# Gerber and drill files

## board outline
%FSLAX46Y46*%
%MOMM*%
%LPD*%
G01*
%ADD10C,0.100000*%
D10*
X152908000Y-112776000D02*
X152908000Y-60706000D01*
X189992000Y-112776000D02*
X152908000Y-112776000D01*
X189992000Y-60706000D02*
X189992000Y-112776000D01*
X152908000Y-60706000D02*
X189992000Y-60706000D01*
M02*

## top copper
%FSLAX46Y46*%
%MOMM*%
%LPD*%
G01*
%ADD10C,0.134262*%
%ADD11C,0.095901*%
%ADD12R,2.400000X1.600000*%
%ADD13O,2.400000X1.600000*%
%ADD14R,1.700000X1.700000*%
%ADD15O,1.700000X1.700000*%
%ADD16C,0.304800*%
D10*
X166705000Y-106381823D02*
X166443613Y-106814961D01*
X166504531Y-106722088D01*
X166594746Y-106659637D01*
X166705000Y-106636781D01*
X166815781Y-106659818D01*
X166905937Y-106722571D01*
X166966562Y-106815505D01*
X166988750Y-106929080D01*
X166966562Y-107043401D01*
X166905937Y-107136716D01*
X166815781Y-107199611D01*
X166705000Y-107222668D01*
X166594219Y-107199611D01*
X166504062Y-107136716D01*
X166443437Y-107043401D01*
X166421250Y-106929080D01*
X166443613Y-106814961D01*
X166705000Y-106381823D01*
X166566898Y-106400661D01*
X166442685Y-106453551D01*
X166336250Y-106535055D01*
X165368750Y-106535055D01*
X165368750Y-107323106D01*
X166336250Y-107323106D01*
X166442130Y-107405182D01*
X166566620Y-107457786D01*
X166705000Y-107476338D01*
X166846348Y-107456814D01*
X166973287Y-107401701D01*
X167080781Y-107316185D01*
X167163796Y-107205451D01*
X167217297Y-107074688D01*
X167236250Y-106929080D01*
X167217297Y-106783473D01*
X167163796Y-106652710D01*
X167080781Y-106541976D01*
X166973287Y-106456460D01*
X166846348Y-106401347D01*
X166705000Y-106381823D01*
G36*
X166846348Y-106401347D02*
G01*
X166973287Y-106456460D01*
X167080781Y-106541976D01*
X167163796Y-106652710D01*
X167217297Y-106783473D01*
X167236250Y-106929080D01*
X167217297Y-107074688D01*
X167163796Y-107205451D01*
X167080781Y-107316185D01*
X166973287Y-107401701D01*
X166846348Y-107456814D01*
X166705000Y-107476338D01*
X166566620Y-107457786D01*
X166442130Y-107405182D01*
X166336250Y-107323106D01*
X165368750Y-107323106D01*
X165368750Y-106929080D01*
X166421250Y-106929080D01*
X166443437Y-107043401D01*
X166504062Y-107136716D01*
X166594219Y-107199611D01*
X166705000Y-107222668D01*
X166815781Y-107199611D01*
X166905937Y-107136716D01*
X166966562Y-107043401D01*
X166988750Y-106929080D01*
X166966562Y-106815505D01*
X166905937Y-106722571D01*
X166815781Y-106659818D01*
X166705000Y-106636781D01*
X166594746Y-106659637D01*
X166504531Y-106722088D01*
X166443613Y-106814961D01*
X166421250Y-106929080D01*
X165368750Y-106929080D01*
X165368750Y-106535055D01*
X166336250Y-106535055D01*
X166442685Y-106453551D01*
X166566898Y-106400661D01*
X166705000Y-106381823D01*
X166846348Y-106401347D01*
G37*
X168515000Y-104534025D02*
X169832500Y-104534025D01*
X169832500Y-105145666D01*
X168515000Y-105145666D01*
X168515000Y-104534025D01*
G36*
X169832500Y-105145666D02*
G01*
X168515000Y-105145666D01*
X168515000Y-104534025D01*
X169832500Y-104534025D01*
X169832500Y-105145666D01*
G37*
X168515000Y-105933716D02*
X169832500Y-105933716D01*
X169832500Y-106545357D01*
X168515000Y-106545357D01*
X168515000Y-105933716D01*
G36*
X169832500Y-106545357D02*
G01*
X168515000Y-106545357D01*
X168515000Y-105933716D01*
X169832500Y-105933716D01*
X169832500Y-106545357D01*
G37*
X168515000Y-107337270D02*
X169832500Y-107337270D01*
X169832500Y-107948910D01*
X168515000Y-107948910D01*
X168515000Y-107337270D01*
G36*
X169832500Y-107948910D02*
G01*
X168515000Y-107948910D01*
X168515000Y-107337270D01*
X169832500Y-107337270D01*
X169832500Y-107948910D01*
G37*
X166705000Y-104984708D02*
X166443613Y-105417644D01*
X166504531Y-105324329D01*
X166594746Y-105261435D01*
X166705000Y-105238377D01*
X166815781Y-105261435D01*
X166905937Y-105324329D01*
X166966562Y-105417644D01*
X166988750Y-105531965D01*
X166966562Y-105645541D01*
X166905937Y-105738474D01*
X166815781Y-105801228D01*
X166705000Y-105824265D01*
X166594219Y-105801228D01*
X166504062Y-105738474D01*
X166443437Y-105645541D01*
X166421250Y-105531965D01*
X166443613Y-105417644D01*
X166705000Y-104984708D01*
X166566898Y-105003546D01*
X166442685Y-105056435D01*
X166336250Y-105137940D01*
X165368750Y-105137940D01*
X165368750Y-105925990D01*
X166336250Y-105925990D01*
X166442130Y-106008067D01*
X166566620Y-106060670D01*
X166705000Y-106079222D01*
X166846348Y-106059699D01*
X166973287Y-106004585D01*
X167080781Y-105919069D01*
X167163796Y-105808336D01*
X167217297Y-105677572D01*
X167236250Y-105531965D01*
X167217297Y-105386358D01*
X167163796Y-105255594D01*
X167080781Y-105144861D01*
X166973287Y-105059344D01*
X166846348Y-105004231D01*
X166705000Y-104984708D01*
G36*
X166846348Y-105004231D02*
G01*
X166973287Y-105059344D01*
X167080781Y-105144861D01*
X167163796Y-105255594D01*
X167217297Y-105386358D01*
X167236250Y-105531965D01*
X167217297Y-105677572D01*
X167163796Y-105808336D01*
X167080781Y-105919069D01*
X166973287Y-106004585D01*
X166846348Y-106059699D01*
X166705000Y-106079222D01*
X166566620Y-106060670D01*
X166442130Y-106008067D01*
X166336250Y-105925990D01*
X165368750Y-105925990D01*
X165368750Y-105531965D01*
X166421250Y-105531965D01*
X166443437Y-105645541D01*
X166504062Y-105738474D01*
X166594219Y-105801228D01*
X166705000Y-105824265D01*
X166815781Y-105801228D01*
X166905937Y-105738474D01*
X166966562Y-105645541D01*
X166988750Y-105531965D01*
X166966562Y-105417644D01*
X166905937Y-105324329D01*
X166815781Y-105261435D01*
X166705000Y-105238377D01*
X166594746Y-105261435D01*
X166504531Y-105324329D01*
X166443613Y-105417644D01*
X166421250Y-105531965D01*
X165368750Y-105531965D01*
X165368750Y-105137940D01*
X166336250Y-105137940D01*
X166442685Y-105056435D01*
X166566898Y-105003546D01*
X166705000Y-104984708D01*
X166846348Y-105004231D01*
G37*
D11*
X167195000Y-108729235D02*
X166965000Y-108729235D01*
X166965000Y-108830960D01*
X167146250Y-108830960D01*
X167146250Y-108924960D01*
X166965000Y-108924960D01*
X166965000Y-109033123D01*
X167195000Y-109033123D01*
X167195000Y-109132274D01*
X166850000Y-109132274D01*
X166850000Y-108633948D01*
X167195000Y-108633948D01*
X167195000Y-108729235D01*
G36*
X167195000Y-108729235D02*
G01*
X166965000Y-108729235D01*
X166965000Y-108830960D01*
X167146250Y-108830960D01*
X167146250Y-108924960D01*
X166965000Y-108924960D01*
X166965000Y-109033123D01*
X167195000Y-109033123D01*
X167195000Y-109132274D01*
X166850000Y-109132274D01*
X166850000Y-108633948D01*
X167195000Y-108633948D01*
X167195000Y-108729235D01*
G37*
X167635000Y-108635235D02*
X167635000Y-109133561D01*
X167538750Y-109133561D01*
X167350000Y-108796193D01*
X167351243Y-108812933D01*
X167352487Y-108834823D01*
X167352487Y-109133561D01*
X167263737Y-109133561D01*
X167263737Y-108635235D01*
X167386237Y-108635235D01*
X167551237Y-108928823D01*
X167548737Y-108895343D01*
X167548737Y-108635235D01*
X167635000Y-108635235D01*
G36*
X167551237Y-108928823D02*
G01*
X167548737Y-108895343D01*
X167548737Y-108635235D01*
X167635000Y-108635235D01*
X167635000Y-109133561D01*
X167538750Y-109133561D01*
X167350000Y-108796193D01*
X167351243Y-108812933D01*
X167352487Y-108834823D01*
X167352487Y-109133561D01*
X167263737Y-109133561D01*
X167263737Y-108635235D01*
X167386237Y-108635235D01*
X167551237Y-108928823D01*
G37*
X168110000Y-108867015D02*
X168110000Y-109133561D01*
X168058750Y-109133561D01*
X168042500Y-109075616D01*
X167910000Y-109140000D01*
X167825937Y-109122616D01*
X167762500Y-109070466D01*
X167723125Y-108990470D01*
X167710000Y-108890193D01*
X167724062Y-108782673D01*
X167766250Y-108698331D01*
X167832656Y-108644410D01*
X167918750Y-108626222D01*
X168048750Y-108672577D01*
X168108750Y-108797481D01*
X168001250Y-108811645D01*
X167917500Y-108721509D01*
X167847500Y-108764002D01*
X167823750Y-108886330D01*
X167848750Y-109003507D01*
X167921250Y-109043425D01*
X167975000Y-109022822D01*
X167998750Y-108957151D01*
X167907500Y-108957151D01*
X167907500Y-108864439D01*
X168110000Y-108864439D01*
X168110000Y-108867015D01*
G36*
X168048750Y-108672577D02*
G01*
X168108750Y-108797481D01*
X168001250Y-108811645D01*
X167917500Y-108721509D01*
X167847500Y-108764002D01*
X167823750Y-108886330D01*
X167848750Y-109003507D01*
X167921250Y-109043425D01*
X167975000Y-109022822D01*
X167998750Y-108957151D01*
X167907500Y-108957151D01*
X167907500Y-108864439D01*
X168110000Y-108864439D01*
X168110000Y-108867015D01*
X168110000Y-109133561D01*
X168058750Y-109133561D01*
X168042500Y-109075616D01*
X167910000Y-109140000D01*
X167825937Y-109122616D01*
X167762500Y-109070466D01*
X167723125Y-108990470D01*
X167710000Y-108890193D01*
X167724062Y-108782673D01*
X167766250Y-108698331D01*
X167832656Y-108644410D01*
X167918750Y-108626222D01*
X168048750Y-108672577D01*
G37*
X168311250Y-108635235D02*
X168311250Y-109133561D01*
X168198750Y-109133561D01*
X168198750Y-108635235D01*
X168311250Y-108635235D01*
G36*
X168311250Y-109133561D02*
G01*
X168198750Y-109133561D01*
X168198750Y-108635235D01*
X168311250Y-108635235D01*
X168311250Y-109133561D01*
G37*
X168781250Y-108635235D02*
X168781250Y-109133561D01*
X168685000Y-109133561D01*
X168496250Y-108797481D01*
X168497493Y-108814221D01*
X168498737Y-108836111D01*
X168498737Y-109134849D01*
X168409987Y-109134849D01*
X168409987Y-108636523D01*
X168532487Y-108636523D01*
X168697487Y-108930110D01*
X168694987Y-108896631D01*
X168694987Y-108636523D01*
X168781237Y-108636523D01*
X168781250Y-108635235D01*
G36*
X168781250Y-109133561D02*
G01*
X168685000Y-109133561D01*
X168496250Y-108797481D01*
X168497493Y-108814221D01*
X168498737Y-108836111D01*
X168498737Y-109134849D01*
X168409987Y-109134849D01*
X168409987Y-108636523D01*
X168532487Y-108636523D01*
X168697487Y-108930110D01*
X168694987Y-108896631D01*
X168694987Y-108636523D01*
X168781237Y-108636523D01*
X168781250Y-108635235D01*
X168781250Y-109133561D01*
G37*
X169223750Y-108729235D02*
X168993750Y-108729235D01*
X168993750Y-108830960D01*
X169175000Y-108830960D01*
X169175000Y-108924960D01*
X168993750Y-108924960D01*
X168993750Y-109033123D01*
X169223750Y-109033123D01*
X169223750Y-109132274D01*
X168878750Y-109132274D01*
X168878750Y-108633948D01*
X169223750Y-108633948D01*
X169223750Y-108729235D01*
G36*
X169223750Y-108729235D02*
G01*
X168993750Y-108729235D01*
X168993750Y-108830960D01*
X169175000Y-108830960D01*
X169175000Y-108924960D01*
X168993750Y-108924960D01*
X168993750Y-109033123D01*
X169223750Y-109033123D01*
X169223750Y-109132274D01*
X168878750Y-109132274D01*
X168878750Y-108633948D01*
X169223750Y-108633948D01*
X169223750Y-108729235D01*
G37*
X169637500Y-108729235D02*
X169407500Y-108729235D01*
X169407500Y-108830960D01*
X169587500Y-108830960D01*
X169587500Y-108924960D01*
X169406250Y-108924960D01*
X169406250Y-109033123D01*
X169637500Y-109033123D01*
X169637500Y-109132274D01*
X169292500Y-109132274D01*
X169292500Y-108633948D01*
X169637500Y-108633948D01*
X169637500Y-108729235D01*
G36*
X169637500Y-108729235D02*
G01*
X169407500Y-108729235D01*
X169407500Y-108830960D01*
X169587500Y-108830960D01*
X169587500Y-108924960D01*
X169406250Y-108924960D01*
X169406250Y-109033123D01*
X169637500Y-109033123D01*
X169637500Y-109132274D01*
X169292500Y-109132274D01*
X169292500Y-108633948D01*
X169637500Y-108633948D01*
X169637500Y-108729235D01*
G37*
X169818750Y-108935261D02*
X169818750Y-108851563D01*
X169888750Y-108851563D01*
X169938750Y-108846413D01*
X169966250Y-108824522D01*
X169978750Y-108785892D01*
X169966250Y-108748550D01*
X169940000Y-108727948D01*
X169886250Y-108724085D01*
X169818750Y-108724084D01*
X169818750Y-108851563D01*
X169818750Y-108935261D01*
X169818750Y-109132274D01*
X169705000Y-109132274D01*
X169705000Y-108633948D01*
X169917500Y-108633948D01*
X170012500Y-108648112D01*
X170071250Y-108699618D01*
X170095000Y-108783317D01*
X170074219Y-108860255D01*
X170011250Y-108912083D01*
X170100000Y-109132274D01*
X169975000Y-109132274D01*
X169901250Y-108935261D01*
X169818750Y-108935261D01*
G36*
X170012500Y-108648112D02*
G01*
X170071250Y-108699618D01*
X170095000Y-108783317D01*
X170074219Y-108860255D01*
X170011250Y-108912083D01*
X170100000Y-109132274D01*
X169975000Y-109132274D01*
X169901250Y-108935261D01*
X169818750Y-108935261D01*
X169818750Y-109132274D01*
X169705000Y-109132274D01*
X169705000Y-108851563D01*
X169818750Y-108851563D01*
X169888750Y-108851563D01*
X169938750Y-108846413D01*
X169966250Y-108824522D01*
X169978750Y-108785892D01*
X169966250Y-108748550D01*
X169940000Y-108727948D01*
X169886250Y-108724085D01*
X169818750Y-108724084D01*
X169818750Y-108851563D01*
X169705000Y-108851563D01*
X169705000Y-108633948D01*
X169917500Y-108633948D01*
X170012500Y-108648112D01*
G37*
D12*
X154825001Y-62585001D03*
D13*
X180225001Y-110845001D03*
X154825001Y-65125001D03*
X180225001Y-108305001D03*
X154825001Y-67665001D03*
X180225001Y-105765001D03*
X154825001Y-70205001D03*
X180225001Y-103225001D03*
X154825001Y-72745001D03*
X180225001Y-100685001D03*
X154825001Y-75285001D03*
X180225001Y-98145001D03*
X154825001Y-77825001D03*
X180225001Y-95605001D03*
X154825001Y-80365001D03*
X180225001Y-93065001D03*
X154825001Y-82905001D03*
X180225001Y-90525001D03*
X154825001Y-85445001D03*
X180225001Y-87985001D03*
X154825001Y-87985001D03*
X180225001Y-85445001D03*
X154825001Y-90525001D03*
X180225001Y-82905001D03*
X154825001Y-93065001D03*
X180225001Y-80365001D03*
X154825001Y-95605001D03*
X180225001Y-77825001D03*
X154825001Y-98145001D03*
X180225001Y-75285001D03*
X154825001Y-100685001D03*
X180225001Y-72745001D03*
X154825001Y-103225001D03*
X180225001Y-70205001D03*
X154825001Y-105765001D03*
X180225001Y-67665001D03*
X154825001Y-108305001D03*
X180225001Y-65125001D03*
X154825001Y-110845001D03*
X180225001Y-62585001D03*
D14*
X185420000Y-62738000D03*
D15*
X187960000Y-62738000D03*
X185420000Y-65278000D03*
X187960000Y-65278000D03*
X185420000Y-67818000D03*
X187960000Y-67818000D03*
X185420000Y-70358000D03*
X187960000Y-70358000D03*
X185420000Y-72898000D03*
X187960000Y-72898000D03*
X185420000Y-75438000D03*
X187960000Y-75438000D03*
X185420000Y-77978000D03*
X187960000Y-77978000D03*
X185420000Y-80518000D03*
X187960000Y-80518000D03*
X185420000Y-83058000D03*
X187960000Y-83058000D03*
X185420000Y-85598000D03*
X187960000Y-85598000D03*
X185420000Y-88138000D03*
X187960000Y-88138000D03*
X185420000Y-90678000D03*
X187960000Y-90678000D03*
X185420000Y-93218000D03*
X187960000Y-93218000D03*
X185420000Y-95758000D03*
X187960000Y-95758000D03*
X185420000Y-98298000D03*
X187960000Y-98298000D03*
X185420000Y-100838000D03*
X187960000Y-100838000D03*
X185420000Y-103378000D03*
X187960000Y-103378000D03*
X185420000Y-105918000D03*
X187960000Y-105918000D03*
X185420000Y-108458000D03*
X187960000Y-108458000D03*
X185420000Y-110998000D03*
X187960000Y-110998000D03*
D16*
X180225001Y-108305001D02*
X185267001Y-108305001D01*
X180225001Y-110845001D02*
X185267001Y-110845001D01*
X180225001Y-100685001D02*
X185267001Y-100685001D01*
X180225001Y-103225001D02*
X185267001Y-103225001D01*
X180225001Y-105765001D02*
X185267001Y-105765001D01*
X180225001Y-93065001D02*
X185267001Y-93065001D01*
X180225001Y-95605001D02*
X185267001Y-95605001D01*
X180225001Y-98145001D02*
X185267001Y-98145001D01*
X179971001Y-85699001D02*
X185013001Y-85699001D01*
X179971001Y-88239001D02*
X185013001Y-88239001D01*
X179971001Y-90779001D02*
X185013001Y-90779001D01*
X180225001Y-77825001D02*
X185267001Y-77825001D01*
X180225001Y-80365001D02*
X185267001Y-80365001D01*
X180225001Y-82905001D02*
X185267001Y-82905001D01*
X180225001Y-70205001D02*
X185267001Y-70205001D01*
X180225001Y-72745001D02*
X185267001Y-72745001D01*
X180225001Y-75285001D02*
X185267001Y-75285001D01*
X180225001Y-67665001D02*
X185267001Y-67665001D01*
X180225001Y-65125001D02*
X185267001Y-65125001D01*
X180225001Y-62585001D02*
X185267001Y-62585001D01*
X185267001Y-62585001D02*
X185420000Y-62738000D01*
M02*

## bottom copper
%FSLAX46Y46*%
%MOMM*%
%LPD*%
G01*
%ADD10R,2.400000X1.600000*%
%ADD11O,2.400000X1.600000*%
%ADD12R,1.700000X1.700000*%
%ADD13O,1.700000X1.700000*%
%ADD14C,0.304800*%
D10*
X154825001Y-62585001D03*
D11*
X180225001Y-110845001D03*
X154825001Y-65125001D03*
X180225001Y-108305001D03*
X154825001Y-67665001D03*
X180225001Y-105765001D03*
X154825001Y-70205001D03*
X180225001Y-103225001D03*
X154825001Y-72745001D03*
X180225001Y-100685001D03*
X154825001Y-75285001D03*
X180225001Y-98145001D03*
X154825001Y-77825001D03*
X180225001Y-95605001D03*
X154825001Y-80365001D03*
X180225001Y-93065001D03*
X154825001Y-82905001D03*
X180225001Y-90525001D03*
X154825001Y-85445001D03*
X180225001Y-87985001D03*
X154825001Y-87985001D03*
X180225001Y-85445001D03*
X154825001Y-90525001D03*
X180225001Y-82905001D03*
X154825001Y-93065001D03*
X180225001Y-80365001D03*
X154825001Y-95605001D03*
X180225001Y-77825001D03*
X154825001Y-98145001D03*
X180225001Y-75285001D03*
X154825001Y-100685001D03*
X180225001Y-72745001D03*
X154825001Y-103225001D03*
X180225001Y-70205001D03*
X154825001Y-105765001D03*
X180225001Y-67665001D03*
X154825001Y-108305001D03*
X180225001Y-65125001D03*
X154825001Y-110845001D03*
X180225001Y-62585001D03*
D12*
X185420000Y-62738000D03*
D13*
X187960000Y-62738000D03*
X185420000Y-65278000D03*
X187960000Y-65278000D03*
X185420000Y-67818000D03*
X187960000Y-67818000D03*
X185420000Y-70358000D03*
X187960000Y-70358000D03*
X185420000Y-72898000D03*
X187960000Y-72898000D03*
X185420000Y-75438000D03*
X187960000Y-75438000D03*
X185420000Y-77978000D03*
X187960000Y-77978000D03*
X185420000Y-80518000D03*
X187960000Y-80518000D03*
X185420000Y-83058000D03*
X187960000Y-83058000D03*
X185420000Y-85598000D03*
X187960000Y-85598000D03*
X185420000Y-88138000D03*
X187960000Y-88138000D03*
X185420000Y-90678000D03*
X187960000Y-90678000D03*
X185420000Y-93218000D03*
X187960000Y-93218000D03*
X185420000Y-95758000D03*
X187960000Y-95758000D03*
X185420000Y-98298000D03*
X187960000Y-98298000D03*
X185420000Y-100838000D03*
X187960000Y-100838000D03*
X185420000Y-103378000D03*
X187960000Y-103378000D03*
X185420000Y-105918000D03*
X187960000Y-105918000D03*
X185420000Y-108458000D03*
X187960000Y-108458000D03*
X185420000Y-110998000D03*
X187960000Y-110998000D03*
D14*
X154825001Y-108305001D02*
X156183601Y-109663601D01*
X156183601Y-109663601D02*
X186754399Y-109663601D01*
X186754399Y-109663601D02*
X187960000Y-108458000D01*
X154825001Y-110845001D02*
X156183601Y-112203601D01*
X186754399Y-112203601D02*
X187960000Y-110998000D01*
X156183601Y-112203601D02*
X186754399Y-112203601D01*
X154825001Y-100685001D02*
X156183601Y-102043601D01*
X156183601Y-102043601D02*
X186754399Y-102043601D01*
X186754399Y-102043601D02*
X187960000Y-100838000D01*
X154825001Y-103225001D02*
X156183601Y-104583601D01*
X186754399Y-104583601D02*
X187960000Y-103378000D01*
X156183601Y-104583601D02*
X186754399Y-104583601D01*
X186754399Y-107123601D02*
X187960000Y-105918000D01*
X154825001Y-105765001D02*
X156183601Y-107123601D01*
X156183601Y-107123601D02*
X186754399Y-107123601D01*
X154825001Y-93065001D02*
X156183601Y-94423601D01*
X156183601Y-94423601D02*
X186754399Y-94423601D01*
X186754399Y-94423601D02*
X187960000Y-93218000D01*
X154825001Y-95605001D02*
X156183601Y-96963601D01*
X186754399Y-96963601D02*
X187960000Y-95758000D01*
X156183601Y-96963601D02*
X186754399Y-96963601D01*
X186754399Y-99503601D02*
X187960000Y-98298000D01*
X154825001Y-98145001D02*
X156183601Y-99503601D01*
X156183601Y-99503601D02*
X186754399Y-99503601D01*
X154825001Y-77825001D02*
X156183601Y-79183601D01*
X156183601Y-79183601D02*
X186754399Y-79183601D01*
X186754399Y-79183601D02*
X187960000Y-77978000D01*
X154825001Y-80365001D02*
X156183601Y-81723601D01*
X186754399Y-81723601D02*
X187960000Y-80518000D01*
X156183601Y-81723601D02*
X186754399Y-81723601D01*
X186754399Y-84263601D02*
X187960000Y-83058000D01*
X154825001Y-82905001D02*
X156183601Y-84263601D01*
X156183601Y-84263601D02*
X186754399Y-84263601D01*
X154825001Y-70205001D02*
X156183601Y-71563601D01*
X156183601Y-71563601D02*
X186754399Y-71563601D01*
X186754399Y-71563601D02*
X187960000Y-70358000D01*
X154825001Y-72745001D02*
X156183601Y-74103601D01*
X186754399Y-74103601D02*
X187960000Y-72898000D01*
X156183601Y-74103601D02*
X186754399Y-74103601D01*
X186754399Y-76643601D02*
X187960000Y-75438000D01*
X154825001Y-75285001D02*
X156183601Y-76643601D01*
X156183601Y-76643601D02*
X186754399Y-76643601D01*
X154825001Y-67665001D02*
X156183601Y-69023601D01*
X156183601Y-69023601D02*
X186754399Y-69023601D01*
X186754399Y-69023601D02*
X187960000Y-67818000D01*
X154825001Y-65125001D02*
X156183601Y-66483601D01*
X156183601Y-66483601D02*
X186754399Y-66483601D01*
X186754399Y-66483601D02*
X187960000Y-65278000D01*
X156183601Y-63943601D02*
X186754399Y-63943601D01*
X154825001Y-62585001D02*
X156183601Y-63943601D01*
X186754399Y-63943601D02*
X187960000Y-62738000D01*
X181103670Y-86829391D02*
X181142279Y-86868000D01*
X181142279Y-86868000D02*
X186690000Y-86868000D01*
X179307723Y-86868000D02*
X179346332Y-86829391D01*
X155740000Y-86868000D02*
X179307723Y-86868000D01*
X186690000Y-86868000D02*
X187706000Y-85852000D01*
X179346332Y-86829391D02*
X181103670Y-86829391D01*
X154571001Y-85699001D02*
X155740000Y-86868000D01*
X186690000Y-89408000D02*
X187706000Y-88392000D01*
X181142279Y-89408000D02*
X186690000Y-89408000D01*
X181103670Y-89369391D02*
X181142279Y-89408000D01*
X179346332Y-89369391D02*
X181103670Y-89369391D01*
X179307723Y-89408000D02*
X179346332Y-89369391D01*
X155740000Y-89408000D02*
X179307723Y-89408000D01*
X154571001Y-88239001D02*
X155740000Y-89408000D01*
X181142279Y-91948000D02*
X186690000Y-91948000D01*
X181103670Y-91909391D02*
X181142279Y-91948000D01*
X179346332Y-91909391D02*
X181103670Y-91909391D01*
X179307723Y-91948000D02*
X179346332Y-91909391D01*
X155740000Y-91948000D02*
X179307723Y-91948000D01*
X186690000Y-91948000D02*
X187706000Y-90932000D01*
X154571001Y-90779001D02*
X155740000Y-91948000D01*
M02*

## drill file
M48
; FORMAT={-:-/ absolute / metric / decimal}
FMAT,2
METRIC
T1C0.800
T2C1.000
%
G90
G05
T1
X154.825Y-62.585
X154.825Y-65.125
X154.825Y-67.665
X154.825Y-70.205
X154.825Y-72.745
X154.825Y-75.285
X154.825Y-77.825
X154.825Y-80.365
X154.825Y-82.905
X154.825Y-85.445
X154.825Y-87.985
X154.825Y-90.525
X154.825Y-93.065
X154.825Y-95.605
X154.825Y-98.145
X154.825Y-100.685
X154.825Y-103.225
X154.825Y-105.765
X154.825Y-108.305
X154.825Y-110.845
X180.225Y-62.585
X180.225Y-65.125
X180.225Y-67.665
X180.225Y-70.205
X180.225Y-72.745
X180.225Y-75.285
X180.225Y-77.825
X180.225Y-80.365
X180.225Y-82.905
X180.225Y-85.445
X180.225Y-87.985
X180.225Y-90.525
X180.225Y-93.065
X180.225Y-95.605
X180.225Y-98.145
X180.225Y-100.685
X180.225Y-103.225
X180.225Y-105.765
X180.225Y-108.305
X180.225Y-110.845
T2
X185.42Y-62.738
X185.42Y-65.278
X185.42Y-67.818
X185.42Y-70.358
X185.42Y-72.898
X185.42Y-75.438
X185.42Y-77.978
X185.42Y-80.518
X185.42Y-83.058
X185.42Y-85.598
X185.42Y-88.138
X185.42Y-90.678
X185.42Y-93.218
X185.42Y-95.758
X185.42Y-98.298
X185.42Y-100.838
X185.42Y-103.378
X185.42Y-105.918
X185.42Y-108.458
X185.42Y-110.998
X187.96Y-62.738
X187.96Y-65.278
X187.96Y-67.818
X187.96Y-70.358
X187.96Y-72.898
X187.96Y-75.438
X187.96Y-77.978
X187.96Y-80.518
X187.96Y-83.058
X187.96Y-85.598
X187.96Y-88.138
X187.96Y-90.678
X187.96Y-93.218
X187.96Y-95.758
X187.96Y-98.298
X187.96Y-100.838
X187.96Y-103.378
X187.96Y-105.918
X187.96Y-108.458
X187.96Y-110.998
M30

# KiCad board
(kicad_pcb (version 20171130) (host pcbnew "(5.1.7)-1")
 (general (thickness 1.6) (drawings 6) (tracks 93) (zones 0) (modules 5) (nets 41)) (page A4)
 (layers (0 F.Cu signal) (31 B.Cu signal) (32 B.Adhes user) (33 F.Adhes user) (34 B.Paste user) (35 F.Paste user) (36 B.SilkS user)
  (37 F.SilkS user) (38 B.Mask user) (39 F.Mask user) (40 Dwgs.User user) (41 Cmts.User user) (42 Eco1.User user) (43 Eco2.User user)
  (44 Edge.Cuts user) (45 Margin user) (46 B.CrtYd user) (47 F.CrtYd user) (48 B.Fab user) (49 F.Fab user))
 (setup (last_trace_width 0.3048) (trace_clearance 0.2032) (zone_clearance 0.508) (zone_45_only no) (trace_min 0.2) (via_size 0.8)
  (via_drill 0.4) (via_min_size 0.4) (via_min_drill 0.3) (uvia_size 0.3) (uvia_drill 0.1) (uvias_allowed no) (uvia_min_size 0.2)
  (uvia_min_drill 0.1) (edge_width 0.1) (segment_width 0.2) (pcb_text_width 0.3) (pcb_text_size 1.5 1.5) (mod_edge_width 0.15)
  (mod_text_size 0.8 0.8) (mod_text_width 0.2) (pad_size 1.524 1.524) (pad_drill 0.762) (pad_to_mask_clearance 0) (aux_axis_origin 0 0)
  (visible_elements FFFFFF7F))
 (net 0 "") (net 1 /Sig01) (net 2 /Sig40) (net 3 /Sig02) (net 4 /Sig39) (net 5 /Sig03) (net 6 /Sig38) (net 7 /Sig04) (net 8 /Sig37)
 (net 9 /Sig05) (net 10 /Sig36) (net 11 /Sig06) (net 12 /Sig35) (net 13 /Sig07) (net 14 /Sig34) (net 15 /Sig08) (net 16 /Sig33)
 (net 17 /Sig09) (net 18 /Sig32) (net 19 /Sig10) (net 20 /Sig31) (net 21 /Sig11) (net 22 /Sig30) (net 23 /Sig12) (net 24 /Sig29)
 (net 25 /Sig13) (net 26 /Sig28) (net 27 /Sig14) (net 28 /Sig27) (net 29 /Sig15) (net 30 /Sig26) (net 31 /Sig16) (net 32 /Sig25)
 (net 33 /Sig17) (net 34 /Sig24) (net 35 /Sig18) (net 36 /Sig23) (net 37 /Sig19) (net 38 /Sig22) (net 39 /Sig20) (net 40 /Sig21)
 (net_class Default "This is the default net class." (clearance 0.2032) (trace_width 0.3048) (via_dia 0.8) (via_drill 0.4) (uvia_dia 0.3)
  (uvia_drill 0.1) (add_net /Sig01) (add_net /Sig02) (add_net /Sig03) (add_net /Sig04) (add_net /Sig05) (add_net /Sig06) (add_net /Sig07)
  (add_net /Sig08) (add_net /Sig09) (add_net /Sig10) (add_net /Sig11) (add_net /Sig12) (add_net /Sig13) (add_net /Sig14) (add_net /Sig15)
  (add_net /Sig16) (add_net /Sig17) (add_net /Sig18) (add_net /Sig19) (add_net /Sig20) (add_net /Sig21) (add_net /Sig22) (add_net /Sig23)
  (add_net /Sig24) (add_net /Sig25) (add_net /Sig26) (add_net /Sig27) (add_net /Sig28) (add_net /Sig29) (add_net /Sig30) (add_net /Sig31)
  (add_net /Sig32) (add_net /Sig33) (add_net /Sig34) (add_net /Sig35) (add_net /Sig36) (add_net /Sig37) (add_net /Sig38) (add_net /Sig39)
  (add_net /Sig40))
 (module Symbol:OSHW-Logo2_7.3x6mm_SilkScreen (layer B.Cu) (at 167.386 106.934 180)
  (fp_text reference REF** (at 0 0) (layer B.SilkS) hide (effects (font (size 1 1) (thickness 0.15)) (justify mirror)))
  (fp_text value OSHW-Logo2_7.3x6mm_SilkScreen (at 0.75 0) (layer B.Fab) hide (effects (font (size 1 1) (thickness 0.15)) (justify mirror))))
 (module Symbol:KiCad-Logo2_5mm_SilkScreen (layer B.Cu) (at 167.386 86.614 180)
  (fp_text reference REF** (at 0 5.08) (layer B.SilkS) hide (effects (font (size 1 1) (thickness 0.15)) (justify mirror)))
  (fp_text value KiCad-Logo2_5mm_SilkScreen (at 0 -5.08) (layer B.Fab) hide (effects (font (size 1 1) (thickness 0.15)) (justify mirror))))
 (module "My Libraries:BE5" (layer F.Cu) (at 165.1 104.14)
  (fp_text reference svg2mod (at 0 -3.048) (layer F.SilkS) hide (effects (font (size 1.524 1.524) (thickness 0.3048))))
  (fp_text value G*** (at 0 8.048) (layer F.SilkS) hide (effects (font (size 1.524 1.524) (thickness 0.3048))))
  (fp_poly
   (pts (xy 1.605 2.241823) (xy 1.343613 2.674961) (xy 1.404531 2.582088) (xy 1.494746 2.519637) (xy 1.605 2.496781) (xy 1.715781 2.519818)
    (xy 1.805937 2.582571) (xy 1.866562 2.675505) (xy 1.88875 2.78908) (xy 1.866562 2.903401) (xy 1.805937 2.996716) (xy 1.715781 3.059611)
    (xy 1.605 3.082668) (xy 1.494219 3.059611) (xy 1.404062 2.996716) (xy 1.343437 2.903401) (xy 1.32125 2.78908) (xy 1.343613 2.674961)
    (xy 1.605 2.241823) (xy 1.466898 2.260661) (xy 1.342685 2.313551) (xy 1.23625 2.395055) (xy 0.26875 2.395055) (xy 0.26875 3.183106)
    (xy 1.23625 3.183106) (xy 1.34213 3.265182) (xy 1.46662 3.317786) (xy 1.605 3.336338) (xy 1.746348 3.316814) (xy 1.873287 3.261701)
    (xy 1.980781 3.176185) (xy 2.063796 3.065451) (xy 2.117297 2.934688) (xy 2.13625 2.78908) (xy 2.117297 2.643473) (xy 2.063796 2.51271)
    (xy 1.980781 2.401976) (xy 1.873287 2.31646) (xy 1.746348 2.261347) (xy 1.605 2.241823))
   (layer F.Cu) (width 0.134262))
  (fp_poly
   (pts (xy 3.415 0.394025) (xy 4.7325 0.394025) (xy 4.7325 1.005666) (xy 3.415 1.005666) (xy 3.415 0.394025)) (layer F.Cu) (width 0.134262))
  (fp_poly
   (pts (xy 3.415 1.793716) (xy 4.7325 1.793716) (xy 4.7325 2.405357) (xy 3.415 2.405357) (xy 3.415 1.793716)) (layer F.Cu) (width 0.134262))
  (fp_poly
   (pts (xy 3.415 3.19727) (xy 4.7325 3.19727) (xy 4.7325 3.80891) (xy 3.415 3.80891) (xy 3.415 3.19727)) (layer F.Cu) (width 0.134262))
  (fp_poly
   (pts (xy 1.605 0.844708) (xy 1.343613 1.277644) (xy 1.404531 1.184329) (xy 1.494746 1.121435) (xy 1.605 1.098377) (xy 1.715781 1.121435)
    (xy 1.805937 1.184329) (xy 1.866562 1.277644) (xy 1.88875 1.391965) (xy 1.866562 1.505541) (xy 1.805937 1.598474) (xy 1.715781 1.661228)
    (xy 1.605 1.684265) (xy 1.494219 1.661228) (xy 1.404062 1.598474) (xy 1.343437 1.505541) (xy 1.32125 1.391965) (xy 1.343613 1.277644)
    (xy 1.605 0.844708) (xy 1.466898 0.863546) (xy 1.342685 0.916435) (xy 1.23625 0.99794) (xy 0.26875 0.99794) (xy 0.26875 1.78599)
    (xy 1.23625 1.78599) (xy 1.34213 1.868067) (xy 1.46662 1.92067) (xy 1.605 1.939222) (xy 1.746348 1.919699) (xy 1.873287 1.864585)
    (xy 1.980781 1.779069) (xy 2.063796 1.668336) (xy 2.117297 1.537572) (xy 2.13625 1.391965) (xy 2.117297 1.246358) (xy 2.063796 1.115594)
    (xy 1.980781 1.004861) (xy 1.873287 0.919344) (xy 1.746348 0.864231) (xy 1.605 0.844708))
   (layer F.Cu) (width 0.134262))
  (fp_poly
   (pts (xy 2.095 4.589235) (xy 1.865 4.589235) (xy 1.865 4.69096) (xy 2.04625 4.69096) (xy 2.04625 4.78496) (xy 1.865 4.78496)
    (xy 1.865 4.893123) (xy 2.095 4.893123) (xy 2.095 4.992274) (xy 1.75 4.992274) (xy 1.75 4.493948) (xy 2.095 4.493948)
    (xy 2.095 4.589235))
   (layer F.Cu) (width 0.095901))
  (fp_poly
   (pts (xy 2.535 4.495235) (xy 2.535 4.993561) (xy 2.43875 4.993561) (xy 2.25 4.656193) (xy 2.251243 4.672933) (xy 2.252487 4.694823)
    (xy 2.252487 4.993561) (xy 2.163737 4.993561) (xy 2.163737 4.495235) (xy 2.286237 4.495235) (xy 2.451237 4.788823)
    (xy 2.448737 4.755343) (xy 2.448737 4.495235) (xy 2.535 4.495235))
   (layer F.Cu) (width 0.095901))
  (fp_poly
   (pts (xy 3.01 4.727015) (xy 3.01 4.993561) (xy 2.95875 4.993561) (xy 2.9425 4.935616) (xy 2.81 5) (xy 2.725937 4.982616)
    (xy 2.6625 4.930466) (xy 2.623125 4.85047) (xy 2.61 4.750193) (xy 2.624062 4.642673) (xy 2.66625 4.558331) (xy 2.732656 4.50441)
    (xy 2.81875 4.486222) (xy 2.94875 4.532577) (xy 3.00875 4.657481) (xy 2.90125 4.671645) (xy 2.8175 4.581509) (xy 2.7475 4.624002)
    (xy 2.72375 4.74633) (xy 2.74875 4.863507) (xy 2.82125 4.903425) (xy 2.875 4.882822) (xy 2.89875 4.817151) (xy 2.8075 4.817151)
    (xy 2.8075 4.724439) (xy 3.01 4.724439) (xy 3.01 4.727015))
   (layer F.Cu) (width 0.095901))
  (fp_poly
   (pts (xy 3.21125 4.495235) (xy 3.21125 4.993561) (xy 3.09875 4.993561) (xy 3.09875 4.495235) (xy 3.21125 4.495235)) (layer F.Cu)
   (width 0.095901))
  (fp_poly
   (pts (xy 3.68125 4.495235) (xy 3.68125 4.993561) (xy 3.585 4.993561) (xy 3.39625 4.657481) (xy 3.397493 4.674221) (xy 3.398737 4.696111)
    (xy 3.398737 4.994849) (xy 3.309987 4.994849) (xy 3.309987 4.496523) (xy 3.432487 4.496523) (xy 3.597487 4.79011) (xy 3.594987 4.756631)
    (xy 3.594987 4.496523) (xy 3.681237 4.496523) (xy 3.68125 4.495235))
   (layer F.Cu) (width 0.095901))
  (fp_poly
   (pts (xy 4.12375 4.589235) (xy 3.89375 4.589235) (xy 3.89375 4.69096) (xy 4.075 4.69096) (xy 4.075 4.78496) (xy 3.89375 4.78496)
    (xy 3.89375 4.893123) (xy 4.12375 4.893123) (xy 4.12375 4.992274) (xy 3.77875 4.992274) (xy 3.77875 4.493948) (xy 4.12375 4.493948)
    (xy 4.12375 4.589235))
   (layer F.Cu) (width 0.095901))
  (fp_poly
   (pts (xy 4.5375 4.589235) (xy 4.3075 4.589235) (xy 4.3075 4.69096) (xy 4.4875 4.69096) (xy 4.4875 4.78496) (xy 4.30625 4.78496)
    (xy 4.30625 4.893123) (xy 4.5375 4.893123) (xy 4.5375 4.992274) (xy 4.1925 4.992274) (xy 4.1925 4.493948) (xy 4.5375 4.493948)
    (xy 4.5375 4.589235))
   (layer F.Cu) (width 0.095901))
  (fp_poly
   (pts (xy 4.71875 4.795261) (xy 4.71875 4.711563) (xy 4.78875 4.711563) (xy 4.83875 4.706413) (xy 4.86625 4.684522) (xy 4.87875 4.645892)
    (xy 4.86625 4.60855) (xy 4.84 4.587948) (xy 4.78625 4.584085) (xy 4.71875 4.584084) (xy 4.71875 4.711563) (xy 4.71875 4.795261)
    (xy 4.71875 4.992274) (xy 4.605 4.992274) (xy 4.605 4.493948) (xy 4.8175 4.493948) (xy 4.9125 4.508112) (xy 4.97125 4.559618)
    (xy 4.995 4.643317) (xy 4.974219 4.720255) (xy 4.91125 4.772083) (xy 5 4.992274) (xy 4.875 4.992274) (xy 4.80125 4.795261)
    (xy 4.71875 4.795261))
   (layer F.Cu) (width 0.095901)))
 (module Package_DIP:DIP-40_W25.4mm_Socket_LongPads (layer F.Cu) (at 154.825001 62.585001)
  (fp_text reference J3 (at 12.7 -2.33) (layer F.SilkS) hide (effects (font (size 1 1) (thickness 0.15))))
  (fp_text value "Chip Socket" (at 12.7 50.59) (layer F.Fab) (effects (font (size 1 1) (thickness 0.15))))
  (pad 1 thru_hole rect (at 0 0) (size 2.4 1.6) (drill 0.8) (layers *.Cu *.Mask) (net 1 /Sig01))
  (pad 21 thru_hole oval (at 25.4 48.26) (size 2.4 1.6) (drill 0.8) (layers *.Cu *.Mask) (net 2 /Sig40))
  (pad 2 thru_hole oval (at 0 2.54) (size 2.4 1.6) (drill 0.8) (layers *.Cu *.Mask) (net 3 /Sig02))
  (pad 22 thru_hole oval (at 25.4 45.72) (size 2.4 1.6) (drill 0.8) (layers *.Cu *.Mask) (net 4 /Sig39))
  (pad 3 thru_hole oval (at 0 5.08) (size 2.4 1.6) (drill 0.8) (layers *.Cu *.Mask) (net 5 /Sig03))
  (pad 23 thru_hole oval (at 25.4 43.18) (size 2.4 1.6) (drill 0.8) (layers *.Cu *.Mask) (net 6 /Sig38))
  (pad 4 thru_hole oval (at 0 7.62) (size 2.4 1.6) (drill 0.8) (layers *.Cu *.Mask) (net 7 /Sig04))
  (pad 24 thru_hole oval (at 25.4 40.64) (size 2.4 1.6) (drill 0.8) (layers *.Cu *.Mask) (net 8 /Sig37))
  (pad 5 thru_hole oval (at 0 10.16) (size 2.4 1.6) (drill 0.8) (layers *.Cu *.Mask) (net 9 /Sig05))
  (pad 25 thru_hole oval (at 25.4 38.1) (size 2.4 1.6) (drill 0.8) (layers *.Cu *.Mask) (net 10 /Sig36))
  (pad 6 thru_hole oval (at 0 12.7) (size 2.4 1.6) (drill 0.8) (layers *.Cu *.Mask) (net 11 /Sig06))
  (pad 26 thru_hole oval (at 25.4 35.56) (size 2.4 1.6) (drill 0.8) (layers *.Cu *.Mask) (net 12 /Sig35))
  (pad 7 thru_hole oval (at 0 15.24) (size 2.4 1.6) (drill 0.8) (layers *.Cu *.Mask) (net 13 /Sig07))
  (pad 27 thru_hole oval (at 25.4 33.02) (size 2.4 1.6) (drill 0.8) (layers *.Cu *.Mask) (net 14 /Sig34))
  (pad 8 thru_hole oval (at 0 17.78) (size 2.4 1.6) (drill 0.8) (layers *.Cu *.Mask) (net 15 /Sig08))
  (pad 28 thru_hole oval (at 25.4 30.48) (size 2.4 1.6) (drill 0.8) (layers *.Cu *.Mask) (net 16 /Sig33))
  (pad 9 thru_hole oval (at 0 20.32) (size 2.4 1.6) (drill 0.8) (layers *.Cu *.Mask) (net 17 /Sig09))
  (pad 29 thru_hole oval (at 25.4 27.94) (size 2.4 1.6) (drill 0.8) (layers *.Cu *.Mask) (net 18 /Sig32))
  (pad 10 thru_hole oval (at 0 22.86) (size 2.4 1.6) (drill 0.8) (layers *.Cu *.Mask) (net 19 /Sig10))
  (pad 30 thru_hole oval (at 25.4 25.4) (size 2.4 1.6) (drill 0.8) (layers *.Cu *.Mask) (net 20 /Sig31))
  (pad 11 thru_hole oval (at 0 25.4) (size 2.4 1.6) (drill 0.8) (layers *.Cu *.Mask) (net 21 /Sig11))
  (pad 31 thru_hole oval (at 25.4 22.86) (size 2.4 1.6) (drill 0.8) (layers *.Cu *.Mask) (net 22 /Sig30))
  (pad 12 thru_hole oval (at 0 27.94) (size 2.4 1.6) (drill 0.8) (layers *.Cu *.Mask) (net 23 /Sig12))
  (pad 32 thru_hole oval (at 25.4 20.32) (size 2.4 1.6) (drill 0.8) (layers *.Cu *.Mask) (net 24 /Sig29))
  (pad 13 thru_hole oval (at 0 30.48) (size 2.4 1.6) (drill 0.8) (layers *.Cu *.Mask) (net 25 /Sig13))
  (pad 33 thru_hole oval (at 25.4 17.78) (size 2.4 1.6) (drill 0.8) (layers *.Cu *.Mask) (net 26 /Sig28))
  (pad 14 thru_hole oval (at 0 33.02) (size 2.4 1.6) (drill 0.8) (layers *.Cu *.Mask) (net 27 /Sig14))
  (pad 34 thru_hole oval (at 25.4 15.24) (size 2.4 1.6) (drill 0.8) (layers *.Cu *.Mask) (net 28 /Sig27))
  (pad 15 thru_hole oval (at 0 35.56) (size 2.4 1.6) (drill 0.8) (layers *.Cu *.Mask) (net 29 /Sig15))
  (pad 35 thru_hole oval (at 25.4 12.7) (size 2.4 1.6) (drill 0.8) (layers *.Cu *.Mask) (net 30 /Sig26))
  (pad 16 thru_hole oval (at 0 38.1) (size 2.4 1.6) (drill 0.8) (layers *.Cu *.Mask) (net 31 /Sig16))
  (pad 36 thru_hole oval (at 25.4 10.16) (size 2.4 1.6) (drill 0.8) (layers *.Cu *.Mask) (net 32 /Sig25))
  (pad 17 thru_hole oval (at 0 40.64) (size 2.4 1.6) (drill 0.8) (layers *.Cu *.Mask) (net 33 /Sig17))
  (pad 37 thru_hole oval (at 25.4 7.62) (size 2.4 1.6) (drill 0.8) (layers *.Cu *.Mask) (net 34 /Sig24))
  (pad 18 thru_hole oval (at 0 43.18) (size 2.4 1.6) (drill 0.8) (layers *.Cu *.Mask) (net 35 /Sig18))
  (pad 38 thru_hole oval (at 25.4 5.08) (size 2.4 1.6) (drill 0.8) (layers *.Cu *.Mask) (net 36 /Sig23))
  (pad 19 thru_hole oval (at 0 45.72) (size 2.4 1.6) (drill 0.8) (layers *.Cu *.Mask) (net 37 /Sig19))
  (pad 39 thru_hole oval (at 25.4 2.54) (size 2.4 1.6) (drill 0.8) (layers *.Cu *.Mask) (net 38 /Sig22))
  (pad 20 thru_hole oval (at 0 48.26) (size 2.4 1.6) (drill 0.8) (layers *.Cu *.Mask) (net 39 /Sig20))
  (pad 40 thru_hole oval (at 25.4 0) (size 2.4 1.6) (drill 0.8) (layers *.Cu *.Mask) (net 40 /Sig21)))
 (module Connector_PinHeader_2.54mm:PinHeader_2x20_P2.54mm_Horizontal (layer F.Cu) (at 185.42 62.738)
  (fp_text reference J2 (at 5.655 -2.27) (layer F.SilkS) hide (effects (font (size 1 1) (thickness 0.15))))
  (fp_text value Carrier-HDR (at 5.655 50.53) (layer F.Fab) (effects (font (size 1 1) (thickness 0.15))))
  (pad 1 thru_hole rect (at 0 0) (size 1.7 1.7) (drill 1) (layers *.Cu *.Mask) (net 40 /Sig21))
  (pad 2 thru_hole oval (at 2.54 0) (size 1.7 1.7) (drill 1) (layers *.Cu *.Mask) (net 1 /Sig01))
  (pad 3 thru_hole oval (at 0 2.54) (size 1.7 1.7) (drill 1) (layers *.Cu *.Mask) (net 38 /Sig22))
  (pad 4 thru_hole oval (at 2.54 2.54) (size 1.7 1.7) (drill 1) (layers *.Cu *.Mask) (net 3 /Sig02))
  (pad 5 thru_hole oval (at 0 5.08) (size 1.7 1.7) (drill 1) (layers *.Cu *.Mask) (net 36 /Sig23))
  (pad 6 thru_hole oval (at 2.54 5.08) (size 1.7 1.7) (drill 1) (layers *.Cu *.Mask) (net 5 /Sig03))
  (pad 7 thru_hole oval (at 0 7.62) (size 1.7 1.7) (drill 1) (layers *.Cu *.Mask) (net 34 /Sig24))
  (pad 8 thru_hole oval (at 2.54 7.62) (size 1.7 1.7) (drill 1) (layers *.Cu *.Mask) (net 7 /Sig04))
  (pad 9 thru_hole oval (at 0 10.16) (size 1.7 1.7) (drill 1) (layers *.Cu *.Mask) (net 32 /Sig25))
  (pad 10 thru_hole oval (at 2.54 10.16) (size 1.7 1.7) (drill 1) (layers *.Cu *.Mask) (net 9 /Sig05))
  (pad 11 thru_hole oval (at 0 12.7) (size 1.7 1.7) (drill 1) (layers *.Cu *.Mask) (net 30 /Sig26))
  (pad 12 thru_hole oval (at 2.54 12.7) (size 1.7 1.7) (drill 1) (layers *.Cu *.Mask) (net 11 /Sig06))
  (pad 13 thru_hole oval (at 0 15.24) (size 1.7 1.7) (drill 1) (layers *.Cu *.Mask) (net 28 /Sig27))
  (pad 14 thru_hole oval (at 2.54 15.24) (size 1.7 1.7) (drill 1) (layers *.Cu *.Mask) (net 13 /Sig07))
  (pad 15 thru_hole oval (at 0 17.78) (size 1.7 1.7) (drill 1) (layers *.Cu *.Mask) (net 26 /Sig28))
  (pad 16 thru_hole oval (at 2.54 17.78) (size 1.7 1.7) (drill 1) (layers *.Cu *.Mask) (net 15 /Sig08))
  (pad 17 thru_hole oval (at 0 20.32) (size 1.7 1.7) (drill 1) (layers *.Cu *.Mask) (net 24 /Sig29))
  (pad 18 thru_hole oval (at 2.54 20.32) (size 1.7 1.7) (drill 1) (layers *.Cu *.Mask) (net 17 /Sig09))
  (pad 19 thru_hole oval (at 0 22.86) (size 1.7 1.7) (drill 1) (layers *.Cu *.Mask) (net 22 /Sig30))
  (pad 20 thru_hole oval (at 2.54 22.86) (size 1.7 1.7) (drill 1) (layers *.Cu *.Mask) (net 19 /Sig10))
  (pad 21 thru_hole oval (at 0 25.4) (size 1.7 1.7) (drill 1) (layers *.Cu *.Mask) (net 20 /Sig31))
  (pad 22 thru_hole oval (at 2.54 25.4) (size 1.7 1.7) (drill 1) (layers *.Cu *.Mask) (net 21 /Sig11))
  (pad 23 thru_hole oval (at 0 27.94) (size 1.7 1.7) (drill 1) (layers *.Cu *.Mask) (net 18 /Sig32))
  (pad 24 thru_hole oval (at 2.54 27.94) (size 1.7 1.7) (drill 1) (layers *.Cu *.Mask) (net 23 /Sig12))
  (pad 25 thru_hole oval (at 0 30.48) (size 1.7 1.7) (drill 1) (layers *.Cu *.Mask) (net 16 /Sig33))
  (pad 26 thru_hole oval (at 2.54 30.48) (size 1.7 1.7) (drill 1) (layers *.Cu *.Mask) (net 25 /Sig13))
  (pad 27 thru_hole oval (at 0 33.02) (size 1.7 1.7) (drill 1) (layers *.Cu *.Mask) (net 14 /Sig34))
  (pad 28 thru_hole oval (at 2.54 33.02) (size 1.7 1.7) (drill 1) (layers *.Cu *.Mask) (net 27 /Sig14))
  (pad 29 thru_hole oval (at 0 35.56) (size 1.7 1.7) (drill 1) (layers *.Cu *.Mask) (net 12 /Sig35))
  (pad 30 thru_hole oval (at 2.54 35.56) (size 1.7 1.7) (drill 1) (layers *.Cu *.Mask) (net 29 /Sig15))
  (pad 31 thru_hole oval (at 0 38.1) (size 1.7 1.7) (drill 1) (layers *.Cu *.Mask) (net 10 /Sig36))
  (pad 32 thru_hole oval (at 2.54 38.1) (size 1.7 1.7) (drill 1) (layers *.Cu *.Mask) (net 31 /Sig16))
  (pad 33 thru_hole oval (at 0 40.64) (size 1.7 1.7) (drill 1) (layers *.Cu *.Mask) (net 8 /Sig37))
  (pad 34 thru_hole oval (at 2.54 40.64) (size 1.7 1.7) (drill 1) (layers *.Cu *.Mask) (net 33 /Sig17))
  (pad 35 thru_hole oval (at 0 43.18) (size 1.7 1.7) (drill 1) (layers *.Cu *.Mask) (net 6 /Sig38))
  (pad 36 thru_hole oval (at 2.54 43.18) (size 1.7 1.7) (drill 1) (layers *.Cu *.Mask) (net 35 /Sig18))
  (pad 37 thru_hole oval (at 0 45.72) (size 1.7 1.7) (drill 1) (layers *.Cu *.Mask) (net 4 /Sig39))
  (pad 38 thru_hole oval (at 2.54 45.72) (size 1.7 1.7) (drill 1) (layers *.Cu *.Mask) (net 37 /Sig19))
  (pad 39 thru_hole oval (at 0 48.26) (size 1.7 1.7) (drill 1) (layers *.Cu *.Mask) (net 2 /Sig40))
  (pad 40 thru_hole oval (at 2.54 48.26) (size 1.7 1.7) (drill 1) (layers *.Cu *.Mask) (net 39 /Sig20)))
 (gr_line (start 152.908 112.776) (end 152.908 60.706) (layer Edge.Cuts) (width 0.1))
 (gr_line (start 189.992 112.776) (end 152.908 112.776) (layer Edge.Cuts) (width 0.1))
 (gr_line (start 189.992 60.706) (end 189.992 112.776) (layer Edge.Cuts) (width 0.1))
 (gr_line (start 152.908 60.706) (end 189.992 60.706) (layer Edge.Cuts) (width 0.1))
 (segment (start 154.825001 108.305001) (end 156.183601 109.663601) (width 0.3048) (layer B.Cu) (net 37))
 (segment (start 156.183601 109.663601) (end 186.754399 109.663601) (width 0.3048) (layer B.Cu) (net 37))
 (segment (start 186.754399 109.663601) (end 187.96 108.458) (width 0.3048) (layer B.Cu) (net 37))
 (segment (start 180.225001 108.305001) (end 185.267001 108.305001) (width 0.3048) (layer F.Cu) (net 4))
 (segment (start 154.825001 110.845001) (end 156.183601 112.203601) (width 0.3048) (layer B.Cu) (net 39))
 (segment (start 186.754399 112.203601) (end 187.96 110.998) (width 0.3048) (layer B.Cu) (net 39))
 (segment (start 156.183601 112.203601) (end 186.754399 112.203601) (width 0.3048) (layer B.Cu) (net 39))
 (segment (start 180.225001 110.845001) (end 185.267001 110.845001) (width 0.3048) (layer F.Cu) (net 2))
 (segment (start 154.825001 100.685001) (end 156.183601 102.043601) (width 0.3048) (layer B.Cu) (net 31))
 (segment (start 156.183601 102.043601) (end 186.754399 102.043601) (width 0.3048) (layer B.Cu) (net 31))
 (segment (start 186.754399 102.043601) (end 187.96 100.838) (width 0.3048) (layer B.Cu) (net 31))
 (segment (start 180.225001 100.685001) (end 185.267001 100.685001) (width 0.3048) (layer F.Cu) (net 10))
 (segment (start 154.825001 103.225001) (end 156.183601 104.583601) (width 0.3048) (layer B.Cu) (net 33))
 (segment (start 186.754399 104.583601) (end 187.96 103.378) (width 0.3048) (layer B.Cu) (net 33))
 (segment (start 156.183601 104.583601) (end 186.754399 104.583601) (width 0.3048) (layer B.Cu) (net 33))
 (segment (start 180.225001 103.225001) (end 185.267001 103.225001) (width 0.3048) (layer F.Cu) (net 8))
 (segment (start 186.754399 107.123601) (end 187.96 105.918) (width 0.3048) (layer B.Cu) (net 35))
 (segment (start 154.825001 105.765001) (end 156.183601 107.123601) (width 0.3048) (layer B.Cu) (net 35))
 (segment (start 156.183601 107.123601) (end 186.754399 107.123601) (width 0.3048) (layer B.Cu) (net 35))
 (segment (start 180.225001 105.765001) (end 185.267001 105.765001) (width 0.3048) (layer F.Cu) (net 6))
 (segment (start 154.825001 93.065001) (end 156.183601 94.423601) (width 0.3048) (layer B.Cu) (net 25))
 (segment (start 156.183601 94.423601) (end 186.754399 94.423601) (width 0.3048) (layer B.Cu) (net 25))
 (segment (start 186.754399 94.423601) (end 187.96 93.218) (width 0.3048) (layer B.Cu) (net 25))
 (segment (start 180.225001 93.065001) (end 185.267001 93.065001) (width 0.3048) (layer F.Cu) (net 16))
 (segment (start 154.825001 95.605001) (end 156.183601 96.963601) (width 0.3048) (layer B.Cu) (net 27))
 (segment (start 186.754399 96.963601) (end 187.96 95.758) (width 0.3048) (layer B.Cu) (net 27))
 (segment (start 156.183601 96.963601) (end 186.754399 96.963601) (width 0.3048) (layer B.Cu) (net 27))
 (segment (start 180.225001 95.605001) (end 185.267001 95.605001) (width 0.3048) (layer F.Cu) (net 14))
 (segment (start 186.754399 99.503601) (end 187.96 98.298) (width 0.3048) (layer B.Cu) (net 29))
 (segment (start 154.825001 98.145001) (end 156.183601 99.503601) (width 0.3048) (layer B.Cu) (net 29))
 (segment (start 156.183601 99.503601) (end 186.754399 99.503601) (width 0.3048) (layer B.Cu) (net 29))
 (segment (start 180.225001 98.145001) (end 185.267001 98.145001) (width 0.3048) (layer F.Cu) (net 12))
 (segment (start 179.971001 85.699001) (end 185.013001 85.699001) (width 0.3048) (layer F.Cu) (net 22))
 (segment (start 179.971001 88.239001) (end 185.013001 88.239001) (width 0.3048) (layer F.Cu) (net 20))
 (segment (start 179.971001 90.779001) (end 185.013001 90.779001) (width 0.3048) (layer F.Cu) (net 18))
 (segment (start 154.825001 77.825001) (end 156.183601 79.183601) (width 0.3048) (layer B.Cu) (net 13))
 (segment (start 156.183601 79.183601) (end 186.754399 79.183601) (width 0.3048) (layer B.Cu) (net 13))
 (segment (start 186.754399 79.183601) (end 187.96 77.978) (width 0.3048) (layer B.Cu) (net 13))
 (segment (start 180.225001 77.825001) (end 185.267001 77.825001) (width 0.3048) (layer F.Cu) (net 28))
 (segment (start 154.825001 80.365001) (end 156.183601 81.723601) (width 0.3048) (layer B.Cu) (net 15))
 (segment (start 186.754399 81.723601) (end 187.96 80.518) (width 0.3048) (layer B.Cu) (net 15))
 (segment (start 156.183601 81.723601) (end 186.754399 81.723601) (width 0.3048) (layer B.Cu) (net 15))
 (segment (start 180.225001 80.365001) (end 185.267001 80.365001) (width 0.3048) (layer F.Cu) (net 26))
 (segment (start 186.754399 84.263601) (end 187.96 83.058) (width 0.3048) (layer B.Cu) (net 17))
 (segment (start 154.825001 82.905001) (end 156.183601 84.263601) (width 0.3048) (layer B.Cu) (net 17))
 (segment (start 156.183601 84.263601) (end 186.754399 84.263601) (width 0.3048) (layer B.Cu) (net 17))
 (segment (start 180.225001 82.905001) (end 185.267001 82.905001) (width 0.3048) (layer F.Cu) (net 24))
 (segment (start 154.825001 70.205001) (end 156.183601 71.563601) (width 0.3048) (layer B.Cu) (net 7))
 (segment (start 156.183601 71.563601) (end 186.754399 71.563601) (width 0.3048) (layer B.Cu) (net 7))
 (segment (start 186.754399 71.563601) (end 187.96 70.358) (width 0.3048) (layer B.Cu) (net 7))
 (segment (start 180.225001 70.205001) (end 185.267001 70.205001) (width 0.3048) (layer F.Cu) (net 34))
 (segment (start 154.825001 72.745001) (end 156.183601 74.103601) (width 0.3048) (layer B.Cu) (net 9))
 (segment (start 186.754399 74.103601) (end 187.96 72.898) (width 0.3048) (layer B.Cu) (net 9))
 (segment (start 156.183601 74.103601) (end 186.754399 74.103601) (width 0.3048) (layer B.Cu) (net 9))
 (segment (start 180.225001 72.745001) (end 185.267001 72.745001) (width 0.3048) (layer F.Cu) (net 32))
 (segment (start 186.754399 76.643601) (end 187.96 75.438) (width 0.3048) (layer B.Cu) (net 11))
 (segment (start 154.825001 75.285001) (end 156.183601 76.643601) (width 0.3048) (layer B.Cu) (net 11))
 (segment (start 156.183601 76.643601) (end 186.754399 76.643601) (width 0.3048) (layer B.Cu) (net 11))
 (segment (start 180.225001 75.285001) (end 185.267001 75.285001) (width 0.3048) (layer F.Cu) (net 30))
 (segment (start 154.825001 67.665001) (end 156.183601 69.023601) (width 0.3048) (layer B.Cu) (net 5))
 (segment (start 156.183601 69.023601) (end 186.754399 69.023601) (width 0.3048) (layer B.Cu) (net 5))
 (segment (start 186.754399 69.023601) (end 187.96 67.818) (width 0.3048) (layer B.Cu) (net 5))
 (segment (start 180.225001 67.665001) (end 185.267001 67.665001) (width 0.3048) (layer F.Cu) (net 36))
 (segment (start 154.825001 65.125001) (end 156.183601 66.483601) (width 0.3048) (layer B.Cu) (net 3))
 (segment (start 156.183601 66.483601) (end 186.754399 66.483601) (width 0.3048) (layer B.Cu) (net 3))
 (segment (start 186.754399 66.483601) (end 187.96 65.278) (width 0.3048) (layer B.Cu) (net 3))
 (segment (start 180.225001 65.125001) (end 185.267001 65.125001) (width 0.3048) (layer F.Cu) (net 38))
 (segment (start 156.183601 63.943601) (end 186.754399 63.943601) (width 0.3048) (layer B.Cu) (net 1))
 (segment (start 154.825001 62.585001) (end 156.183601 63.943601) (width 0.3048) (layer B.Cu) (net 1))
 (segment (start 186.754399 63.943601) (end 187.96 62.738) (width 0.3048) (layer B.Cu) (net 1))
 (segment (start 180.225001 62.585001) (end 185.267001 62.585001) (width 0.3048) (layer F.Cu) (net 40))
 (segment (start 185.267001 62.585001) (end 185.42 62.738) (width 0.3048) (layer F.Cu) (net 40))
 (segment (start 181.10367 86.829391) (end 181.142279 86.868) (width 0.3048) (layer B.Cu) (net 19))
 (segment (start 181.142279 86.868) (end 186.69 86.868) (width 0.3048) (layer B.Cu) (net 19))
 (segment (start 179.307723 86.868) (end 179.346332 86.829391) (width 0.3048) (layer B.Cu) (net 19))
 (segment (start 155.74 86.868) (end 179.307723 86.868) (width 0.3048) (layer B.Cu) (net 19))
 (segment (start 186.69 86.868) (end 187.706 85.852) (width 0.3048) (layer B.Cu) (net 19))
 (segment (start 179.346332 86.829391) (end 181.10367 86.829391) (width 0.3048) (layer B.Cu) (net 19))
 (segment (start 154.571001 85.699001) (end 155.74 86.868) (width 0.3048) (layer B.Cu) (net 19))
 (segment (start 186.69 89.408) (end 187.706 88.392) (width 0.3048) (layer B.Cu) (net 21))
 (segment (start 181.142279 89.408) (end 186.69 89.408) (width 0.3048) (layer B.Cu) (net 21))
 (segment (start 181.10367 89.369391) (end 181.142279 89.408) (width 0.3048) (layer B.Cu) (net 21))
 (segment (start 179.346332 89.369391) (end 181.10367 89.369391) (width 0.3048) (layer B.Cu) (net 21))
 (segment (start 179.307723 89.408) (end 179.346332 89.369391) (width 0.3048) (layer B.Cu) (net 21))
 (segment (start 155.74 89.408) (end 179.307723 89.408) (width 0.3048) (layer B.Cu) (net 21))
 (segment (start 154.571001 88.239001) (end 155.74 89.408) (width 0.3048) (layer B.Cu) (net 21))
 (segment (start 181.142279 91.948) (end 186.69 91.948) (width 0.3048) (layer B.Cu) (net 23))
 (segment (start 181.10367 91.909391) (end 181.142279 91.948) (width 0.3048) (layer B.Cu) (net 23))
 (segment (start 179.346332 91.909391) (end 181.10367 91.909391) (width 0.3048) (layer B.Cu) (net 23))
 (segment (start 179.307723 91.948) (end 179.346332 91.909391) (width 0.3048) (layer B.Cu) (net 23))
 (segment (start 155.74 91.948) (end 179.307723 91.948) (width 0.3048) (layer B.Cu) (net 23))
 (segment (start 186.69 91.948) (end 187.706 90.932) (width 0.3048) (layer B.Cu) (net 23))
 (segment (start 154.571001 90.779001) (end 155.74 91.948) (width 0.3048) (layer B.Cu) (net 23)))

